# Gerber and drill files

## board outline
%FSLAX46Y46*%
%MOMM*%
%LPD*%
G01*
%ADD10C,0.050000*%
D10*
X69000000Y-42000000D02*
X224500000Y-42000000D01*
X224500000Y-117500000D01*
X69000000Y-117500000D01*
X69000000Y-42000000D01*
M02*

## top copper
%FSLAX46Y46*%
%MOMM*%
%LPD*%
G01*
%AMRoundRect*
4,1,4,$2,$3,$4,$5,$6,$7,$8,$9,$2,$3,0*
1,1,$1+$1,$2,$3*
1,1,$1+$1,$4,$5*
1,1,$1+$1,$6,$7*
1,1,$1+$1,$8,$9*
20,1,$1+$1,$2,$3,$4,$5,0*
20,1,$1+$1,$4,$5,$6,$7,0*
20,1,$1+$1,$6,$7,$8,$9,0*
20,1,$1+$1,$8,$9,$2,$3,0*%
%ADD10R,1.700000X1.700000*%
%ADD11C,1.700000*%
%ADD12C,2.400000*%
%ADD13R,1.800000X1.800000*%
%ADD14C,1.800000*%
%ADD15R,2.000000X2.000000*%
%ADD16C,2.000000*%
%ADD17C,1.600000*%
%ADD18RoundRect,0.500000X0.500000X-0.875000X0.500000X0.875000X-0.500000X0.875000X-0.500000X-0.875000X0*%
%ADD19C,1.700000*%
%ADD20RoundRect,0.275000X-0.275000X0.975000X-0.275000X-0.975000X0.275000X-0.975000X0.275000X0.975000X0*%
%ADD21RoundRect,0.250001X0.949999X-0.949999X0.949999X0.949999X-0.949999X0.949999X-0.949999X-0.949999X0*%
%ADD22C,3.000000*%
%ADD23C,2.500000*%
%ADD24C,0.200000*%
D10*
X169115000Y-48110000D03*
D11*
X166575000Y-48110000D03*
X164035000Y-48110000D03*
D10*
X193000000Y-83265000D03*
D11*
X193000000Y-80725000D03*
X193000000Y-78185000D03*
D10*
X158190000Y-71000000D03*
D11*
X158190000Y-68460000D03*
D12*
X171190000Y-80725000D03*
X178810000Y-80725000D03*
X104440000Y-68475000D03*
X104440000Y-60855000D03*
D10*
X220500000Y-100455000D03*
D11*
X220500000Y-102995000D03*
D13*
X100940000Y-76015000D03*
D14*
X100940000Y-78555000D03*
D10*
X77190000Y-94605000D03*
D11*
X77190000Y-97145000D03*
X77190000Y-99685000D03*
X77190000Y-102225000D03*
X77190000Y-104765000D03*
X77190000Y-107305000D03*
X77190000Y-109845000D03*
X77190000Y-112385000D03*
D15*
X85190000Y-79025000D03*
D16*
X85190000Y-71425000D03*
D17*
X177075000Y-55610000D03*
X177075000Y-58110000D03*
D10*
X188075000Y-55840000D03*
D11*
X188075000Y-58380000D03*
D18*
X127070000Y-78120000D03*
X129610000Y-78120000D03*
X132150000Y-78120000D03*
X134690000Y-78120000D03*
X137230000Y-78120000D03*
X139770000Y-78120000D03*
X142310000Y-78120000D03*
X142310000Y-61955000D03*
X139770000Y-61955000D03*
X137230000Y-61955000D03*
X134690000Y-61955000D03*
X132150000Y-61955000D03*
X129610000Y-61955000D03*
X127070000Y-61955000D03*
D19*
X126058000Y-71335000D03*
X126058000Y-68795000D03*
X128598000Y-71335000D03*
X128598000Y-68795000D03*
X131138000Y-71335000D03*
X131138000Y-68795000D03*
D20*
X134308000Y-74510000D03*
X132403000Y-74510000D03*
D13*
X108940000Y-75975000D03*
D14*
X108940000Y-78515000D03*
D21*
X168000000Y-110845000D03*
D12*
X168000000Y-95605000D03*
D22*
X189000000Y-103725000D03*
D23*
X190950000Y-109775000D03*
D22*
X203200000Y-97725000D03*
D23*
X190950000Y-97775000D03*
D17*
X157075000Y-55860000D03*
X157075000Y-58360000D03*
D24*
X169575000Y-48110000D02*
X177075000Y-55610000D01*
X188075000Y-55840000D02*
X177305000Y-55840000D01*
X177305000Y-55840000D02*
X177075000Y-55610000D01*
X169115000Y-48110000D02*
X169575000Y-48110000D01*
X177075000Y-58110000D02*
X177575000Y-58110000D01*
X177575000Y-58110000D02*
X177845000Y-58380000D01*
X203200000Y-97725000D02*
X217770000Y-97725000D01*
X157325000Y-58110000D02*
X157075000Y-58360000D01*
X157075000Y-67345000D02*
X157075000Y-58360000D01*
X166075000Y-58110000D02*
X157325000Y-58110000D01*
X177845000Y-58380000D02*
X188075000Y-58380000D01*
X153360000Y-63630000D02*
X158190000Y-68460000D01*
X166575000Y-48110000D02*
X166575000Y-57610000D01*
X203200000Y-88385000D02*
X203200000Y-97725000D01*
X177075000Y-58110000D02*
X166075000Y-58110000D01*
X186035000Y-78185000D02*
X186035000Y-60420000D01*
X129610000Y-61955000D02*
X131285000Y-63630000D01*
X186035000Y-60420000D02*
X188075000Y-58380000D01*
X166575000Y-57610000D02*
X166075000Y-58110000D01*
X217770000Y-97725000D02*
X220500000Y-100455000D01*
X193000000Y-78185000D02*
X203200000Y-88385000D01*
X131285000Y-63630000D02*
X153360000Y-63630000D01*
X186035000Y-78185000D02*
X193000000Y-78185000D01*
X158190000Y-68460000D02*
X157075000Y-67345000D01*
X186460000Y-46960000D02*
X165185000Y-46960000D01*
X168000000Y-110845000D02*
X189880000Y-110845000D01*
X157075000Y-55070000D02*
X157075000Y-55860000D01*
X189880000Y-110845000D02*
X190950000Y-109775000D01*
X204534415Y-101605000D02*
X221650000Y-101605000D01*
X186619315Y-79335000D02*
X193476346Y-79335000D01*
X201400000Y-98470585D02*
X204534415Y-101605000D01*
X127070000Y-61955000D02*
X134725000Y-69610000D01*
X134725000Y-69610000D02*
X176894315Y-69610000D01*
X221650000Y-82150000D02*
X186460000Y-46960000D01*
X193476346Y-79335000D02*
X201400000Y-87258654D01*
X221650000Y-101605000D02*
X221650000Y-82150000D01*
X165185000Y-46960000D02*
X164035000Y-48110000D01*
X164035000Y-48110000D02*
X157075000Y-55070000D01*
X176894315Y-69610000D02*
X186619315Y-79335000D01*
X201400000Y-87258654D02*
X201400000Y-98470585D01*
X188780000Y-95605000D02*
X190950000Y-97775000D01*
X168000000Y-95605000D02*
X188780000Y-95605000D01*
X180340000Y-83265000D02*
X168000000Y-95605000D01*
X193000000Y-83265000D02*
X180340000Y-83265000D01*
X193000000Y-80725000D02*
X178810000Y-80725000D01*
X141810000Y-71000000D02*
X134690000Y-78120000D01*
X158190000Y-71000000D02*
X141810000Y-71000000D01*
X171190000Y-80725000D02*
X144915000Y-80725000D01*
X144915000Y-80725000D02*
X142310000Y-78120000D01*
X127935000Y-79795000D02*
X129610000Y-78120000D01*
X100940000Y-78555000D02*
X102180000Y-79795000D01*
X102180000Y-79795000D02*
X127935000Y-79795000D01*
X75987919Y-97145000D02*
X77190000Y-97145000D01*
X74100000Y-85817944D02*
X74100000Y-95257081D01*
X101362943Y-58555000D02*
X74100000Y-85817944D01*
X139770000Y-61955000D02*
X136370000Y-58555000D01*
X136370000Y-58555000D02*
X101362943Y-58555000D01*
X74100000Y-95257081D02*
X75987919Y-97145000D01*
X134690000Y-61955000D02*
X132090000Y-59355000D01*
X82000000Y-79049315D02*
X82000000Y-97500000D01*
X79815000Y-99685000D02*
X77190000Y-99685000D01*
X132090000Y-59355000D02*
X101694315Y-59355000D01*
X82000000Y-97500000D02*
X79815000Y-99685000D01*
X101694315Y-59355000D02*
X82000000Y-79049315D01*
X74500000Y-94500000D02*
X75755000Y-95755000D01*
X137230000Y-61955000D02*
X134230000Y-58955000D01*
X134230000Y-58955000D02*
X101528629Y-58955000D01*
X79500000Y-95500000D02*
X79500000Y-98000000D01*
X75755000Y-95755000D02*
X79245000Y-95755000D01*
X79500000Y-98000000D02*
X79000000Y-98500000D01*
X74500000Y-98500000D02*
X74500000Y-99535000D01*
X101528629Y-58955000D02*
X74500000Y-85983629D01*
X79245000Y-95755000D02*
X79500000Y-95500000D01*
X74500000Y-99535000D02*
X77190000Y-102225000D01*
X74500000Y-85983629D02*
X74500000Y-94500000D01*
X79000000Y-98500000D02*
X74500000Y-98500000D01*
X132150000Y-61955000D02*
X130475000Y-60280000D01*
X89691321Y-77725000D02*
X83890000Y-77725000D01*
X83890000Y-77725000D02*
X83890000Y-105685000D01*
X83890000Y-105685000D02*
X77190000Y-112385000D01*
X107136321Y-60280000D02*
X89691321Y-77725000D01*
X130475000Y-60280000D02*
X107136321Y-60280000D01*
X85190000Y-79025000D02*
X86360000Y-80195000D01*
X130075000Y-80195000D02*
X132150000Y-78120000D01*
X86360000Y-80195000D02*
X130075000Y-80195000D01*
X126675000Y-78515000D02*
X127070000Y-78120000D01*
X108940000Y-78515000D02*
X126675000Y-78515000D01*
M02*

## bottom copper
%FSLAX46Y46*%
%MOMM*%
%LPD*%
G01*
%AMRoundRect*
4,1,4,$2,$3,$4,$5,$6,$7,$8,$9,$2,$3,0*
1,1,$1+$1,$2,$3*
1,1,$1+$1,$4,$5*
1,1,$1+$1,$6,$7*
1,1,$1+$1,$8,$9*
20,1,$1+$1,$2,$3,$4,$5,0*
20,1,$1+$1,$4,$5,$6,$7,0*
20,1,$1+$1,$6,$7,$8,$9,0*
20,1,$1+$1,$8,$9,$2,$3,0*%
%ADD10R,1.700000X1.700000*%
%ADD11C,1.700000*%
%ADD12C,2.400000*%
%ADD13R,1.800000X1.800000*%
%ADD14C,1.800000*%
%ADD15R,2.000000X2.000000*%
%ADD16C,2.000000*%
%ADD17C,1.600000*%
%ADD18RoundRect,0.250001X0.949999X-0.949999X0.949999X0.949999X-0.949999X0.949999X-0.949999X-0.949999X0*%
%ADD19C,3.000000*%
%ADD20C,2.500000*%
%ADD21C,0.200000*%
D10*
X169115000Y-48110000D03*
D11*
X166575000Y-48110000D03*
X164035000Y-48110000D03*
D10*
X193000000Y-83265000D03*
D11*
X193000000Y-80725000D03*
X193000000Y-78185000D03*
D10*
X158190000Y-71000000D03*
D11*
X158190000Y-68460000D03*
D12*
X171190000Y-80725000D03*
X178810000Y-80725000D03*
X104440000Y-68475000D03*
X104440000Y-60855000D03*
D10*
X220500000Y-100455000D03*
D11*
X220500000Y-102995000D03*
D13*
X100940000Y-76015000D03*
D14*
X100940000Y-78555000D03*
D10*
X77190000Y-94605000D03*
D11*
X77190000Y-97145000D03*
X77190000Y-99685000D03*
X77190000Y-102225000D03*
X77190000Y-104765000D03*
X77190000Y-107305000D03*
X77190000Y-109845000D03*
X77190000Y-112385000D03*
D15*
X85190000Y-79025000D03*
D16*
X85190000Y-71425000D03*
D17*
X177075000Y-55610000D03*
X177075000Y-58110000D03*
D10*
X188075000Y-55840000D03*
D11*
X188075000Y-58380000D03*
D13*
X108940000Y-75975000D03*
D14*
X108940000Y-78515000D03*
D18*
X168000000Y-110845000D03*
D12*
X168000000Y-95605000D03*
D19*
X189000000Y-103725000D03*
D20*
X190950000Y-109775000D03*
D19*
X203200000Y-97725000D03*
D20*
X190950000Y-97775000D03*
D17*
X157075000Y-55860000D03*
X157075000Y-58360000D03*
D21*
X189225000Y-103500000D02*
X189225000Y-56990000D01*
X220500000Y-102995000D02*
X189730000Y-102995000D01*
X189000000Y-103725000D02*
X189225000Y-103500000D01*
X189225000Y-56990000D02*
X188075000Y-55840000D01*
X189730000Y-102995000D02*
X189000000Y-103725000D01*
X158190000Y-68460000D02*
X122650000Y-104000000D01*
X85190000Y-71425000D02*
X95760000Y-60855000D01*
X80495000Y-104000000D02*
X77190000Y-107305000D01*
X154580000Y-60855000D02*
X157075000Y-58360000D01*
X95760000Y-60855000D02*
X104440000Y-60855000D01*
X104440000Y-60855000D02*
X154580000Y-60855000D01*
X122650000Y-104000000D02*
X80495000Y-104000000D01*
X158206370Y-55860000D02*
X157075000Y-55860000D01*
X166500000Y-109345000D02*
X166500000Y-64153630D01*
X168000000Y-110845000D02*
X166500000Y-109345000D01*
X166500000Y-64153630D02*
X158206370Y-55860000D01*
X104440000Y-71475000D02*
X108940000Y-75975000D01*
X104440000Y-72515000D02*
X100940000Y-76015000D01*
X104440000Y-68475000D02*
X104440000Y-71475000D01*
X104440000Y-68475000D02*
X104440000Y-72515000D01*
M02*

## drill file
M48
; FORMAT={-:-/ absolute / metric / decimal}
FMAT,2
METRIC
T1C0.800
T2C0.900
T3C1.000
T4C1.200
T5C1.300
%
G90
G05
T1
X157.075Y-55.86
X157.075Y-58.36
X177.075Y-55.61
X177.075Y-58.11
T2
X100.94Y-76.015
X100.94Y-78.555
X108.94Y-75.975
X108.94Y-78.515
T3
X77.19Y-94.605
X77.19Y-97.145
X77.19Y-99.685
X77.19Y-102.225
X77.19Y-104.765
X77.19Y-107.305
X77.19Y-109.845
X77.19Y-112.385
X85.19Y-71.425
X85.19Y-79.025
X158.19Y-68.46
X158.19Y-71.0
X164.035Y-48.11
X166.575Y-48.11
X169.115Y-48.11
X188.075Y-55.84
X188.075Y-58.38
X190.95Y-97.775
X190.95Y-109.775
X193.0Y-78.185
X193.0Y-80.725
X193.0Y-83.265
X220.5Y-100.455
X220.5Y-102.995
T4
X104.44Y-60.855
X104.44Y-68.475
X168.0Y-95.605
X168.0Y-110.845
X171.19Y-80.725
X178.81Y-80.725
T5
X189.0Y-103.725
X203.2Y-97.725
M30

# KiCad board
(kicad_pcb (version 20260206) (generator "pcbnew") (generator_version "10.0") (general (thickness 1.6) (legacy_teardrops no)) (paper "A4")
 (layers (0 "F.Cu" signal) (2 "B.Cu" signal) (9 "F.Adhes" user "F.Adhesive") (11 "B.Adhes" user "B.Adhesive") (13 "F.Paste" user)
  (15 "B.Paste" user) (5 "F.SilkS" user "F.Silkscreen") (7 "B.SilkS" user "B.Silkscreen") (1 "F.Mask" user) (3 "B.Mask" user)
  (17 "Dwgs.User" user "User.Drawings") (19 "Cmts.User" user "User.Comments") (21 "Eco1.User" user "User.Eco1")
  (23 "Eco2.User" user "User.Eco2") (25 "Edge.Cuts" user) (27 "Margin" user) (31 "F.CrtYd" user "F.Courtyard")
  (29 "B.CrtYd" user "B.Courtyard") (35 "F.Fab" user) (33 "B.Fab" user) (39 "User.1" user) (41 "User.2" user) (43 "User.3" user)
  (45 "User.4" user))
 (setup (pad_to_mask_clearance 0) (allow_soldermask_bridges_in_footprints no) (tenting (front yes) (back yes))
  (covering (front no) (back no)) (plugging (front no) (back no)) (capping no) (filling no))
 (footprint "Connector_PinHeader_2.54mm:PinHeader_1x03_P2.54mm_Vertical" (layer "F.Cu") (at 169.115 48.11 -90)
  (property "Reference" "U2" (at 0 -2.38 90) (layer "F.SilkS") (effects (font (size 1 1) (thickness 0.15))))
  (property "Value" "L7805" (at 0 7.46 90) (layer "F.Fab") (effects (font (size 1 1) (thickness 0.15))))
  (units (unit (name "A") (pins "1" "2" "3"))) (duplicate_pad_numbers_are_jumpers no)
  (pad "1" thru_hole rect (at 0 0 270) (size 1.7 1.7) (drill 1) (layers "*.Cu" "*.Mask") (remove_unused_layers no) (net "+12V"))
  (pad "2" thru_hole circle (at 0 2.54 270) (size 1.7 1.7) (drill 1) (layers "*.Cu" "*.Mask") (remove_unused_layers no) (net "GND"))
  (pad "3" thru_hole circle (at 0 5.08 270) (size 1.7 1.7) (drill 1) (layers "*.Cu" "*.Mask") (remove_unused_layers no) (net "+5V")))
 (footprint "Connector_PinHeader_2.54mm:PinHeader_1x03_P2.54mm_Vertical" (layer "F.Cu") (at 193 83.265 180)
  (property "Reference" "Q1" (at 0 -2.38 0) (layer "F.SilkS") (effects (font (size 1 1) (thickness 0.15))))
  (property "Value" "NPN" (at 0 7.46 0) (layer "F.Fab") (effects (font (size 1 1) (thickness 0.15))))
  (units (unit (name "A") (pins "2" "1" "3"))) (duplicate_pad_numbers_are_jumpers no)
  (pad "1" thru_hole rect (at 0 0 180) (size 1.7 1.7) (drill 1) (layers "*.Cu" "*.Mask") (remove_unused_layers no) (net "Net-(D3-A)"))
  (pad "2" thru_hole circle (at 0 2.54 180) (size 1.7 1.7) (drill 1) (layers "*.Cu" "*.Mask") (remove_unused_layers no) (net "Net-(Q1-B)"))
  (pad "3" thru_hole circle (at 0 5.08 180) (size 1.7 1.7) (drill 1) (layers "*.Cu" "*.Mask") (remove_unused_layers no) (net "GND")))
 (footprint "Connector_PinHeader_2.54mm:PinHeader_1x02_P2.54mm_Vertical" (layer "F.Cu") (at 158.19 71 180)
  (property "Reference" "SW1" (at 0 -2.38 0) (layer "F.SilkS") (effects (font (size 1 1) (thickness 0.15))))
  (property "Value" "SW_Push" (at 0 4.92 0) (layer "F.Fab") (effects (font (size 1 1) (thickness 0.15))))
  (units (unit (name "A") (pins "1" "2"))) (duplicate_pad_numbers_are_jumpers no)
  (pad "1" thru_hole rect (at 0 0 180) (size 1.7 1.7) (drill 1) (layers "*.Cu" "*.Mask") (remove_unused_layers no) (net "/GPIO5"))
  (pad "2" thru_hole circle (at 0 2.54 180) (size 1.7 1.7) (drill 1) (layers "*.Cu" "*.Mask") (remove_unused_layers no) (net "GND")))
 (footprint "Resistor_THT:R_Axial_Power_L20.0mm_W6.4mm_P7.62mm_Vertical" (layer "F.Cu") (at 171.19 80.725)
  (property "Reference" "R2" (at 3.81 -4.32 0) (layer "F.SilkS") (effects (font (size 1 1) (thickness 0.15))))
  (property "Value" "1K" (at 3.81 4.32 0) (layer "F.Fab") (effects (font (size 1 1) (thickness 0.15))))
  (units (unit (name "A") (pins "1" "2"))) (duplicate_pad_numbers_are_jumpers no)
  (pad "1" thru_hole circle (at 0 0) (size 2.4 2.4) (drill 1.2) (layers "*.Cu" "*.Mask") (remove_unused_layers no) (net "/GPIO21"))
  (pad "2" thru_hole circle (at 7.62 0) (size 2.4 2.4) (drill 1.2) (layers "*.Cu" "*.Mask") (remove_unused_layers no) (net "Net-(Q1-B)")))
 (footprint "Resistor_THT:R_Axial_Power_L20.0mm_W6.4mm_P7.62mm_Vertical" (layer "F.Cu") (at 104.44 68.475 90)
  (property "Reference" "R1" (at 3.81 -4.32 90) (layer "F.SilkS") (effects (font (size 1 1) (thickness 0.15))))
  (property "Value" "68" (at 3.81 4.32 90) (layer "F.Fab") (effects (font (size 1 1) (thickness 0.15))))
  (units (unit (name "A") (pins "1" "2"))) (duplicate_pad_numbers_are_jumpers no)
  (pad "1" thru_hole circle (at 0 0 90) (size 2.4 2.4) (drill 1.2) (layers "*.Cu" "*.Mask") (remove_unused_layers no) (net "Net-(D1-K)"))
  (pad "2" thru_hole circle (at 7.62 0 90) (size 2.4 2.4) (drill 1.2) (layers "*.Cu" "*.Mask") (remove_unused_layers no) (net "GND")))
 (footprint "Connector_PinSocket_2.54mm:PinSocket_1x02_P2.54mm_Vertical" (layer "F.Cu") (at 220.5 100.455)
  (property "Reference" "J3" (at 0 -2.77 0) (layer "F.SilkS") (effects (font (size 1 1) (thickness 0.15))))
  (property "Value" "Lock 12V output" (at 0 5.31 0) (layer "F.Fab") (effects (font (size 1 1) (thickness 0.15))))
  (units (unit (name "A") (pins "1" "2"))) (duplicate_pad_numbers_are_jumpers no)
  (pad "1" thru_hole rect (at 0 0) (size 1.7 1.7) (drill 1) (layers "*.Cu" "*.Mask") (remove_unused_layers no) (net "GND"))
  (pad "2" thru_hole circle (at 0 2.54) (size 1.7 1.7) (drill 1) (layers "*.Cu" "*.Mask") (remove_unused_layers no) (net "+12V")))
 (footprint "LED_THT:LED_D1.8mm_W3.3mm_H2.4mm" (layer "F.Cu") (at 100.94 76.015 -90)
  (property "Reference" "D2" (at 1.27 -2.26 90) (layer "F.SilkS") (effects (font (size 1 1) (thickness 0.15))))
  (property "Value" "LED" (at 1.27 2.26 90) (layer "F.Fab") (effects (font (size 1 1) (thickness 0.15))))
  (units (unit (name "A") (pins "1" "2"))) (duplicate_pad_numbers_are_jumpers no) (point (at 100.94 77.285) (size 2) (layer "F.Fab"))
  (pad "1" thru_hole rect (at 0 0 270) (size 1.8 1.8) (drill 0.9) (layers "*.Cu" "*.Mask") (remove_unused_layers no) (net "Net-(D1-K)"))
  (pad "2" thru_hole circle (at 2.54 0 270) (size 1.8 1.8) (drill 0.9) (layers "*.Cu" "*.Mask") (remove_unused_layers no) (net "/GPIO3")))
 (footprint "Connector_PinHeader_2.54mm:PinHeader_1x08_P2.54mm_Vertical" (layer "F.Cu") (at 77.19 94.605)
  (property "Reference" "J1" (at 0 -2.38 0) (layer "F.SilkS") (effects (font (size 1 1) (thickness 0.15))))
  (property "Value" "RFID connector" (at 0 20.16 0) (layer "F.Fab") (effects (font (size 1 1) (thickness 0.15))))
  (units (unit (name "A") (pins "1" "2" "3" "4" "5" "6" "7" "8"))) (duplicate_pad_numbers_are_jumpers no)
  (pad "1" thru_hole rect (at 0 0) (size 1.7 1.7) (drill 1) (layers "*.Cu" "*.Mask") (remove_unused_layers no)
   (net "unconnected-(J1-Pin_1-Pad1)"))
  (pad "2" thru_hole circle (at 0 2.54) (size 1.7 1.7) (drill 1) (layers "*.Cu" "*.Mask") (remove_unused_layers no) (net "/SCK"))
  (pad "3" thru_hole circle (at 0 5.08) (size 1.7 1.7) (drill 1) (layers "*.Cu" "*.Mask") (remove_unused_layers no) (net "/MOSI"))
  (pad "4" thru_hole circle (at 0 7.62) (size 1.7 1.7) (drill 1) (layers "*.Cu" "*.Mask") (remove_unused_layers no) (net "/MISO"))
  (pad "5" thru_hole circle (at 0 10.16) (size 1.7 1.7) (drill 1) (layers "*.Cu" "*.Mask") (remove_unused_layers no)
   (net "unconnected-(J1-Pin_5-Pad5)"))
  (pad "6" thru_hole circle (at 0 12.7) (size 1.7 1.7) (drill 1) (layers "*.Cu" "*.Mask") (remove_unused_layers no) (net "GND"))
  (pad "7" thru_hole circle (at 0 15.24) (size 1.7 1.7) (drill 1) (layers "*.Cu" "*.Mask") (remove_unused_layers no)
   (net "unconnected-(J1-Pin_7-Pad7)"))
  (pad "8" thru_hole circle (at 0 17.78) (size 1.7 1.7) (drill 1) (layers "*.Cu" "*.Mask") (remove_unused_layers no) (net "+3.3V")))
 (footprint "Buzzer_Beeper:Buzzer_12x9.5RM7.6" (layer "F.Cu") (at 85.19 79.025 90)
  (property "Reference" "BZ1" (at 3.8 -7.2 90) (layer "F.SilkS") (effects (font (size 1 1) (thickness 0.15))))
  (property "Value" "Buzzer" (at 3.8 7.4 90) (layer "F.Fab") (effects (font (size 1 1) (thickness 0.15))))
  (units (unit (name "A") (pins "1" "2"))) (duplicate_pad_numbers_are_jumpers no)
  (pad "1" thru_hole rect (at 0 0 90) (size 2 2) (drill 1) (layers "*.Cu" "*.Mask") (remove_unused_layers no) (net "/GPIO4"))
  (pad "2" thru_hole circle (at 7.6 0 90) (size 2 2) (drill 1) (layers "*.Cu" "*.Mask") (remove_unused_layers no) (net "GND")))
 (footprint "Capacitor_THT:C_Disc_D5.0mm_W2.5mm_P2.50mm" (layer "F.Cu") (at 177.075 55.61 -90)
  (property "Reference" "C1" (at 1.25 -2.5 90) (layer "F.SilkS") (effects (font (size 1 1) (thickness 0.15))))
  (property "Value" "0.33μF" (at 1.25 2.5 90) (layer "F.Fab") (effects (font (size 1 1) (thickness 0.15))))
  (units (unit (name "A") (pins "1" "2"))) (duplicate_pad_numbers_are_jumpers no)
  (pad "1" thru_hole circle (at 0 0 270) (size 1.6 1.6) (drill 0.8) (layers "*.Cu" "*.Mask") (remove_unused_layers no) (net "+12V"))
  (pad "2" thru_hole circle (at 2.5 0 270) (size 1.6 1.6) (drill 0.8) (layers "*.Cu" "*.Mask") (remove_unused_layers no) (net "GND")))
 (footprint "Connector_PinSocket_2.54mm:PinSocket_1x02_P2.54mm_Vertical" (layer "F.Cu") (at 188.075 55.84)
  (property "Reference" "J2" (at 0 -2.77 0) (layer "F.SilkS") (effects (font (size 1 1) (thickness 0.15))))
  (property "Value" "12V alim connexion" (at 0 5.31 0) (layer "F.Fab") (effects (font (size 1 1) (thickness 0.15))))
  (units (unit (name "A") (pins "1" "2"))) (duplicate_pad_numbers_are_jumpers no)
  (pad "1" thru_hole rect (at 0 0) (size 1.7 1.7) (drill 1) (layers "*.Cu" "*.Mask") (remove_unused_layers no) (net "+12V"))
  (pad "2" thru_hole circle (at 0 2.54) (size 1.7 1.7) (drill 1) (layers "*.Cu" "*.Mask") (remove_unused_layers no) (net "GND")))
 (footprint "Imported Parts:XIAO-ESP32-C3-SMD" (layer "F.Cu") (at 145.19 78.955 90)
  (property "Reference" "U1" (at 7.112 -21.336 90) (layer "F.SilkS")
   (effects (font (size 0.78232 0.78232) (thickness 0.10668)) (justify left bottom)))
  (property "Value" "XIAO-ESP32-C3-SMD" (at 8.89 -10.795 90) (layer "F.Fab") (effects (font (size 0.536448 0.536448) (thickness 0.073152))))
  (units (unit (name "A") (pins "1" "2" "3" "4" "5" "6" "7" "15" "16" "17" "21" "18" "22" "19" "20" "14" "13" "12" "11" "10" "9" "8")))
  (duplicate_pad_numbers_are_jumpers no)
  (pad "1" smd roundrect (at 0.835 -18.12 90) (size 2.75 2) (layers "F.Cu" "F.Mask" "F.Paste") (roundrect_rratio 0.25) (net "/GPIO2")
   (solder_mask_margin 0.0508) (thermal_bridge_angle 45))
  (pad "2" smd roundrect (at 0.835 -15.58 90) (size 2.75 2) (layers "F.Cu" "F.Mask" "F.Paste") (roundrect_rratio 0.25) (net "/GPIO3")
   (solder_mask_margin 0.0508) (thermal_bridge_angle 45))
  (pad "3" smd roundrect (at 0.835 -13.04 90) (size 2.75 2) (layers "F.Cu" "F.Mask" "F.Paste") (roundrect_rratio 0.25) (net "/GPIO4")
   (solder_mask_margin 0.0508) (thermal_bridge_angle 45))
  (pad "4" smd roundrect (at 0.835 -10.5 90) (size 2.75 2) (layers "F.Cu" "F.Mask" "F.Paste") (roundrect_rratio 0.25) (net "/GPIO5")
   (solder_mask_margin 0.0508) (thermal_bridge_angle 45))
  (pad "5" smd roundrect (at 0.835 -7.96 90) (size 2.75 2) (layers "F.Cu" "F.Mask" "F.Paste") (roundrect_rratio 0.25)
   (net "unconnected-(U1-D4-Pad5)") (solder_mask_margin 0.0508) (thermal_bridge_angle 45))
  (pad "6" smd roundrect (at 0.835 -5.42 90) (size 2.75 2) (layers "F.Cu" "F.Mask" "F.Paste") (roundrect_rratio 0.25)
   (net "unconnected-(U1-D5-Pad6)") (solder_mask_margin 0.0508) (thermal_bridge_angle 45))
  (pad "7" smd roundrect (at 0.835 -2.88 90) (size 2.75 2) (layers "F.Cu" "F.Mask" "F.Paste") (roundrect_rratio 0.25) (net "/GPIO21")
   (solder_mask_margin 0.0508) (thermal_bridge_angle 45))
  (pad "8" smd roundrect (at 17 -2.88 90) (size 2.75 2) (layers "F.Cu" "F.Mask" "F.Paste") (roundrect_rratio 0.25)
   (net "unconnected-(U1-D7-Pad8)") (solder_mask_margin 0.0508) (thermal_bridge_angle 45))
  (pad "9" smd roundrect (at 17 -5.42 90) (size 2.75 2) (layers "F.Cu" "F.Mask" "F.Paste") (roundrect_rratio 0.25) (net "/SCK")
   (solder_mask_margin 0.0508) (thermal_bridge_angle 45))
  (pad "10" smd roundrect (at 17 -7.96 90) (size 2.75 2) (layers "F.Cu" "F.Mask" "F.Paste") (roundrect_rratio 0.25) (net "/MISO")
   (solder_mask_margin 0.0508) (thermal_bridge_angle 45))
  (pad "11" smd roundrect (at 17 -10.5 90) (size 2.75 2) (layers "F.Cu" "F.Mask" "F.Paste") (roundrect_rratio 0.25) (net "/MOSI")
   (solder_mask_margin 0.0508) (thermal_bridge_angle 45))
  (pad "12" smd roundrect (at 17 -13.04 90) (size 2.75 2) (layers "F.Cu" "F.Mask" "F.Paste") (roundrect_rratio 0.25) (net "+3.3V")
   (solder_mask_margin 0.0508) (thermal_bridge_angle 45))
  (pad "13" smd roundrect (at 17 -15.58 90) (size 2.75 2) (layers "F.Cu" "F.Mask" "F.Paste") (roundrect_rratio 0.25) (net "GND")
   (solder_mask_margin 0.0508) (thermal_bridge_angle 45))
  (pad "14" smd roundrect (at 17 -18.12 90) (size 2.75 2) (layers "F.Cu" "F.Mask" "F.Paste") (roundrect_rratio 0.25) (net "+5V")
   (solder_mask_margin 0.0508) (thermal_bridge_angle 45))
  (pad "15" smd circle (at 7.62 -19.132 90) (size 1.7 1.7) (layers "F.Cu" "F.Mask" "F.Paste") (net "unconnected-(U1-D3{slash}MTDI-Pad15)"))
  (pad "16" smd circle (at 10.16 -19.132 90) (size 1.7 1.7) (layers "F.Cu" "F.Mask" "F.Paste") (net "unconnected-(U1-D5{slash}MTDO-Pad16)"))
  (pad "17" smd circle (at 7.62 -16.592 90) (size 1.7 1.7) (layers "F.Cu" "F.Mask" "F.Paste") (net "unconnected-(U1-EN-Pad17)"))
  (pad "18" smd circle (at 10.16 -16.592 90) (size 1.7 1.7) (layers "F.Cu" "F.Mask" "F.Paste") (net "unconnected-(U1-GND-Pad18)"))
  (pad "19" smd circle (at 7.62 -14.052 90) (size 1.7 1.7) (layers "F.Cu" "F.Mask" "F.Paste") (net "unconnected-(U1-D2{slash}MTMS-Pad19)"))
  (pad "20" smd circle (at 10.16 -14.052 90) (size 1.7 1.7) (layers "F.Cu" "F.Mask" "F.Paste") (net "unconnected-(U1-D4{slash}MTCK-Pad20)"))
  (pad "21" smd roundrect (at 4.445 -10.882 270) (size 2.5 1.1) (layers "F.Cu" "F.Mask" "F.Paste") (roundrect_rratio 0.25)
   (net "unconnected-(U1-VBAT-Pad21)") (thermal_bridge_angle 45))
  (pad "22" smd roundrect (at 4.445 -12.787 270) (size 2.5 1.1) (layers "F.Cu" "F.Mask" "F.Paste") (roundrect_rratio 0.25)
   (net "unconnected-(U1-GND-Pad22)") (thermal_bridge_angle 45)))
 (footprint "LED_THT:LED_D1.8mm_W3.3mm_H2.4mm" (layer "F.Cu") (at 108.94 75.975 -90)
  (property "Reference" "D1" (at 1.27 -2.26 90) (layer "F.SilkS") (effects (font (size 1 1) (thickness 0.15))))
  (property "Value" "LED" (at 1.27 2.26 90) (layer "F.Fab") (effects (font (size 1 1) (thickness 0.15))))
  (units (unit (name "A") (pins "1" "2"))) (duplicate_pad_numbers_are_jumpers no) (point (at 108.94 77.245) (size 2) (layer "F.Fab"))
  (pad "1" thru_hole rect (at 0 0 270) (size 1.8 1.8) (drill 0.9) (layers "*.Cu" "*.Mask") (remove_unused_layers no) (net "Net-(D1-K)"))
  (pad "2" thru_hole circle (at 2.54 0 270) (size 1.8 1.8) (drill 0.9) (layers "*.Cu" "*.Mask") (remove_unused_layers no) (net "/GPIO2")))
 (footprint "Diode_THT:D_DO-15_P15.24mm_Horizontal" (layer "F.Cu") (at 168 110.845 90)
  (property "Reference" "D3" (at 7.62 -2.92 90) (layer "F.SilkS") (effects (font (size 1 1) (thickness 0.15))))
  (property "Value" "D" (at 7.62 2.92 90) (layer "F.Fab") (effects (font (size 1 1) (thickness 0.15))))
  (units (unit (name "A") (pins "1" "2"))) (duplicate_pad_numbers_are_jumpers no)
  (pad "1" thru_hole roundrect (at 0 0 90) (size 2.4 2.4) (drill 1.2) (layers "*.Cu" "*.Mask") (remove_unused_layers no)
   (roundrect_rratio 0.104167) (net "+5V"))
  (pad "2" thru_hole circle (at 15.24 0 90) (size 2.4 2.4) (drill 1.2) (layers "*.Cu" "*.Mask") (remove_unused_layers no) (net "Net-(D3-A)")))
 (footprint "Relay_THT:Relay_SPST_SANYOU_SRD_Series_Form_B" (layer "F.Cu") (at 189 103.725)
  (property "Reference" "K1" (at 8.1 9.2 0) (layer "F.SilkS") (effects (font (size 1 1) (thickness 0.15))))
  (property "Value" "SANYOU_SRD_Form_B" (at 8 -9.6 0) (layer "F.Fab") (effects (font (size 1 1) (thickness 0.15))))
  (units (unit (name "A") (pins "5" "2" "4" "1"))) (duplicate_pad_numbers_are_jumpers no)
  (pad "1" thru_hole circle (at 0 0 90) (size 3 3) (drill 1.3) (layers "*.Cu" "*.Mask") (remove_unused_layers no) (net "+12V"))
  (pad "2" thru_hole circle (at 1.95 6.05 90) (size 2.5 2.5) (drill 1) (layers "*.Cu" "*.Mask") (remove_unused_layers no) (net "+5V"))
  (pad "4" thru_hole circle (at 14.2 -6 90) (size 3 3) (drill 1.3) (layers "*.Cu" "*.Mask") (remove_unused_layers no) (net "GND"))
  (pad "5" thru_hole circle (at 1.95 -5.95 90) (size 2.5 2.5) (drill 1) (layers "*.Cu" "*.Mask") (remove_unused_layers no)
   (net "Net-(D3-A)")))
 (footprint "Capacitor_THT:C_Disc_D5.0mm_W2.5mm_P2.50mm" (layer "F.Cu") (at 157.075 55.86 -90)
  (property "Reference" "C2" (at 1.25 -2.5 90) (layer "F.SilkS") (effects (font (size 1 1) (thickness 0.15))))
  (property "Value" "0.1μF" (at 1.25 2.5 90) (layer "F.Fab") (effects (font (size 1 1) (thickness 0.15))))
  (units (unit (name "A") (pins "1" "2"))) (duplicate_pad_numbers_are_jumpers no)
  (pad "1" thru_hole circle (at 0 0 270) (size 1.6 1.6) (drill 0.8) (layers "*.Cu" "*.Mask") (remove_unused_layers no) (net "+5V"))
  (pad "2" thru_hole circle (at 2.5 0 270) (size 1.6 1.6) (drill 0.8) (layers "*.Cu" "*.Mask") (remove_unused_layers no) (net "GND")))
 (gr_rect (start 69 42) (end 224.5 117.5) (stroke (width 0.05) (type default)) (fill no) (layer "Edge.Cuts"))
 (segment (start 169.575 48.11) (end 177.075 55.61) (width 0.2) (layer "F.Cu") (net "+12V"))
 (segment (start 188.075 55.84) (end 177.305 55.84) (width 0.2) (layer "F.Cu") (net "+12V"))
 (segment (start 177.305 55.84) (end 177.075 55.61) (width 0.2) (layer "F.Cu") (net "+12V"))
 (segment (start 169.115 48.11) (end 169.575 48.11) (width 0.2) (layer "F.Cu") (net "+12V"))
 (segment (start 189.225 103.5) (end 189.225 56.99) (width 0.2) (layer "B.Cu") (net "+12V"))
 (segment (start 220.5 102.995) (end 189.73 102.995) (width 0.2) (layer "B.Cu") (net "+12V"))
 (segment (start 189 103.725) (end 189.225 103.5) (width 0.2) (layer "B.Cu") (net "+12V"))
 (segment (start 189.225 56.99) (end 188.075 55.84) (width 0.2) (layer "B.Cu") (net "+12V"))
 (segment (start 189.73 102.995) (end 189 103.725) (width 0.2) (layer "B.Cu") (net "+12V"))
 (segment (start 177.075 58.11) (end 177.575 58.11) (width 0.2) (layer "F.Cu") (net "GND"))
 (segment (start 177.575 58.11) (end 177.845 58.38) (width 0.2) (layer "F.Cu") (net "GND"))
 (segment (start 203.2 97.725) (end 217.77 97.725) (width 0.2) (layer "F.Cu") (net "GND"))
 (segment (start 157.325 58.11) (end 157.075 58.36) (width 0.2) (layer "F.Cu") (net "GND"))
 (segment (start 157.075 67.345) (end 157.075 58.36) (width 0.2) (layer "F.Cu") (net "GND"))
 (segment (start 166.075 58.11) (end 157.325 58.11) (width 0.2) (layer "F.Cu") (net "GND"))
 (segment (start 177.845 58.38) (end 188.075 58.38) (width 0.2) (layer "F.Cu") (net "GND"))
 (segment (start 153.36 63.63) (end 158.19 68.46) (width 0.2) (layer "F.Cu") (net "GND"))
 (segment (start 166.575 48.11) (end 166.575 57.61) (width 0.2) (layer "F.Cu") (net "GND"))
 (segment (start 203.2 88.385) (end 203.2 97.725) (width 0.2) (layer "F.Cu") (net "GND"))
 (segment (start 177.075 58.11) (end 166.075 58.11) (width 0.2) (layer "F.Cu") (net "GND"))
 (segment (start 186.035 78.185) (end 186.035 60.42) (width 0.2) (layer "F.Cu") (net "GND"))
 (segment (start 129.61 61.955) (end 131.285 63.63) (width 0.2) (layer "F.Cu") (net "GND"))
 (segment (start 186.035 60.42) (end 188.075 58.38) (width 0.2) (layer "F.Cu") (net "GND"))
 (segment (start 166.575 57.61) (end 166.075 58.11) (width 0.2) (layer "F.Cu") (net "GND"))
 (segment (start 217.77 97.725) (end 220.5 100.455) (width 0.2) (layer "F.Cu") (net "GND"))
 (segment (start 193 78.185) (end 203.2 88.385) (width 0.2) (layer "F.Cu") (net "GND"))
 (segment (start 131.285 63.63) (end 153.36 63.63) (width 0.2) (layer "F.Cu") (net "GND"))
 (segment (start 186.035 78.185) (end 193 78.185) (width 0.2) (layer "F.Cu") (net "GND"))
 (segment (start 158.19 68.46) (end 157.075 67.345) (width 0.2) (layer "F.Cu") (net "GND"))
 (segment (start 158.19 68.46) (end 122.65 104) (width 0.2) (layer "B.Cu") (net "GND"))
 (segment (start 85.19 71.425) (end 95.76 60.855) (width 0.2) (layer "B.Cu") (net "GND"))
 (segment (start 80.495 104) (end 77.19 107.305) (width 0.2) (layer "B.Cu") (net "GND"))
 (segment (start 154.58 60.855) (end 157.075 58.36) (width 0.2) (layer "B.Cu") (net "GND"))
 (segment (start 95.76 60.855) (end 104.44 60.855) (width 0.2) (layer "B.Cu") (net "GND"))
 (segment (start 104.44 60.855) (end 154.58 60.855) (width 0.2) (layer "B.Cu") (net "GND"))
 (segment (start 122.65 104) (end 80.495 104) (width 0.2) (layer "B.Cu") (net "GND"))
 (segment (start 186.46 46.96) (end 165.185 46.96) (width 0.2) (layer "F.Cu") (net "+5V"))
 (segment (start 168 110.845) (end 189.88 110.845) (width 0.2) (layer "F.Cu") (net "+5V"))
 (segment (start 157.075 55.07) (end 157.075 55.86) (width 0.2) (layer "F.Cu") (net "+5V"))
 (segment (start 189.88 110.845) (end 190.95 109.775) (width 0.2) (layer "F.Cu") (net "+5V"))
 (segment (start 204.534415 101.605) (end 221.65 101.605) (width 0.2) (layer "F.Cu") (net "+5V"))
 (segment (start 186.619315 79.335) (end 193.476346 79.335) (width 0.2) (layer "F.Cu") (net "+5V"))
 (segment (start 201.4 98.470585) (end 204.534415 101.605) (width 0.2) (layer "F.Cu") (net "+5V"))
 (segment (start 127.07 61.955) (end 134.725 69.61) (width 0.2) (layer "F.Cu") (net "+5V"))
 (segment (start 134.725 69.61) (end 176.894315 69.61) (width 0.2) (layer "F.Cu") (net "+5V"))
 (segment (start 221.65 82.15) (end 186.46 46.96) (width 0.2) (layer "F.Cu") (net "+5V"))
 (segment (start 193.476346 79.335) (end 201.4 87.258654) (width 0.2) (layer "F.Cu") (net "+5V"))
 (segment (start 221.65 101.605) (end 221.65 82.15) (width 0.2) (layer "F.Cu") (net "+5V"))
 (segment (start 165.185 46.96) (end 164.035 48.11) (width 0.2) (layer "F.Cu") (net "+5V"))
 (segment (start 164.035 48.11) (end 157.075 55.07) (width 0.2) (layer "F.Cu") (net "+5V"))
 (segment (start 176.894315 69.61) (end 186.619315 79.335) (width 0.2) (layer "F.Cu") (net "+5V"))
 (segment (start 201.4 87.258654) (end 201.4 98.470585) (width 0.2) (layer "F.Cu") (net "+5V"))
 (segment (start 158.20637 55.86) (end 157.075 55.86) (width 0.2) (layer "B.Cu") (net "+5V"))
 (segment (start 166.5 109.345) (end 166.5 64.15363) (width 0.2) (layer "B.Cu") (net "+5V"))
 (segment (start 168 110.845) (end 166.5 109.345) (width 0.2) (layer "B.Cu") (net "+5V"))
 (segment (start 166.5 64.15363) (end 158.20637 55.86) (width 0.2) (layer "B.Cu") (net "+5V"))
 (segment (start 188.78 95.605) (end 190.95 97.775) (width 0.2) (layer "F.Cu") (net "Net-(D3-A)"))
 (segment (start 168 95.605) (end 188.78 95.605) (width 0.2) (layer "F.Cu") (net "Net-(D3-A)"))
 (segment (start 180.34 83.265) (end 168 95.605) (width 0.2) (layer "F.Cu") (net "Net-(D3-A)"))
 (segment (start 193 83.265) (end 180.34 83.265) (width 0.2) (layer "F.Cu") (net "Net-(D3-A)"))
 (segment (start 193 80.725) (end 178.81 80.725) (width 0.2) (layer "F.Cu") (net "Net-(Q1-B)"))
 (segment (start 141.81 71) (end 134.69 78.12) (width 0.2) (layer "F.Cu") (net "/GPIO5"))
 (segment (start 158.19 71) (end 141.81 71) (width 0.2) (layer "F.Cu") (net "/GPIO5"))
 (segment (start 171.19 80.725) (end 144.915 80.725) (width 0.2) (layer "F.Cu") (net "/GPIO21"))
 (segment (start 144.915 80.725) (end 142.31 78.12) (width 0.2) (layer "F.Cu") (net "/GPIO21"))
 (segment (start 104.44 71.475) (end 108.94 75.975) (width 0.2) (layer "B.Cu") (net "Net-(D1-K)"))
 (segment (start 104.44 72.515) (end 100.94 76.015) (width 0.2) (layer "B.Cu") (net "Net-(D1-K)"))
 (segment (start 104.44 68.475) (end 104.44 71.475) (width 0.2) (layer "B.Cu") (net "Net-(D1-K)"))
 (segment (start 104.44 68.475) (end 104.44 72.515) (width 0.2) (layer "B.Cu") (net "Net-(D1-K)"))
 (segment (start 127.935 79.795) (end 129.61 78.12) (width 0.2) (layer "F.Cu") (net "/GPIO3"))
 (segment (start 100.94 78.555) (end 102.18 79.795) (width 0.2) (layer "F.Cu") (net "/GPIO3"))
 (segment (start 102.18 79.795) (end 127.935 79.795) (width 0.2) (layer "F.Cu") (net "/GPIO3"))
 (segment (start 75.987919 97.145) (end 77.19 97.145) (width 0.2) (layer "F.Cu") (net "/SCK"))
 (segment (start 74.1 85.817944) (end 74.1 95.257081) (width 0.2) (layer "F.Cu") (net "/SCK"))
 (segment (start 101.362943 58.555) (end 74.1 85.817944) (width 0.2) (layer "F.Cu") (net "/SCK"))
 (segment (start 139.77 61.955) (end 136.37 58.555) (width 0.2) (layer "F.Cu") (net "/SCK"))
 (segment (start 136.37 58.555) (end 101.362943 58.555) (width 0.2) (layer "F.Cu") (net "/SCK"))
 (segment (start 74.1 95.257081) (end 75.987919 97.145) (width 0.2) (layer "F.Cu") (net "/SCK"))
 (segment (start 134.69 61.955) (end 132.09 59.355) (width 0.2) (layer "F.Cu") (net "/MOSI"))
 (segment (start 82 79.049315) (end 82 97.5) (width 0.2) (layer "F.Cu") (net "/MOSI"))
 (segment (start 79.815 99.685) (end 77.19 99.685) (width 0.2) (layer "F.Cu") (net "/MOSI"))
 (segment (start 132.09 59.355) (end 101.694315 59.355) (width 0.2) (layer "F.Cu") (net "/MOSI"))
 (segment (start 82 97.5) (end 79.815 99.685) (width 0.2) (layer "F.Cu") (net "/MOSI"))
 (segment (start 101.694315 59.355) (end 82 79.049315) (width 0.2) (layer "F.Cu") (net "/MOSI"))
 (segment (start 74.5 94.5) (end 75.755 95.755) (width 0.2) (layer "F.Cu") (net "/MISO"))
 (segment (start 137.23 61.955) (end 134.23 58.955) (width 0.2) (layer "F.Cu") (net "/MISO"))
 (segment (start 134.23 58.955) (end 101.528629 58.955) (width 0.2) (layer "F.Cu") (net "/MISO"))
 (segment (start 79.5 95.5) (end 79.5 98) (width 0.2) (layer "F.Cu") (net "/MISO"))
 (segment (start 75.755 95.755) (end 79.245 95.755) (width 0.2) (layer "F.Cu") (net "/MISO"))
 (segment (start 79.5 98) (end 79 98.5) (width 0.2) (layer "F.Cu") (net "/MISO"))
 (segment (start 74.5 98.5) (end 74.5 99.535) (width 0.2) (layer "F.Cu") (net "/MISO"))
 (segment (start 101.528629 58.955) (end 74.5 85.983629) (width 0.2) (layer "F.Cu") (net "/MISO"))
 (segment (start 79.245 95.755) (end 79.5 95.5) (width 0.2) (layer "F.Cu") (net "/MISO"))
 (segment (start 74.5 99.535) (end 77.19 102.225) (width 0.2) (layer "F.Cu") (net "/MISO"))
 (segment (start 74.5 85.983629) (end 74.5 94.5) (width 0.2) (layer "F.Cu") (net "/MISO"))
 (segment (start 79 98.5) (end 74.5 98.5) (width 0.2) (layer "F.Cu") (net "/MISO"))
 (segment (start 132.15 61.955) (end 130.475 60.28) (width 0.2) (layer "F.Cu") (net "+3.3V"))
 (segment (start 89.691321 77.725) (end 83.89 77.725) (width 0.2) (layer "F.Cu") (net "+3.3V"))
 (segment (start 83.89 77.725) (end 83.89 105.685) (width 0.2) (layer "F.Cu") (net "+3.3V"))
 (segment (start 83.89 105.685) (end 77.19 112.385) (width 0.2) (layer "F.Cu") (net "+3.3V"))
 (segment (start 107.136321 60.28) (end 89.691321 77.725) (width 0.2) (layer "F.Cu") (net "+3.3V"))
 (segment (start 130.475 60.28) (end 107.136321 60.28) (width 0.2) (layer "F.Cu") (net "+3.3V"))
 (segment (start 85.19 79.025) (end 86.36 80.195) (width 0.2) (layer "F.Cu") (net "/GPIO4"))
 (segment (start 130.075 80.195) (end 132.15 78.12) (width 0.2) (layer "F.Cu") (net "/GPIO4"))
 (segment (start 86.36 80.195) (end 130.075 80.195) (width 0.2) (layer "F.Cu") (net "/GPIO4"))
 (segment (start 126.675 78.515) (end 127.07 78.12) (width 0.2) (layer "F.Cu") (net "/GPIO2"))
 (segment (start 108.94 78.515) (end 126.675 78.515) (width 0.2) (layer "F.Cu") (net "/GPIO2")))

